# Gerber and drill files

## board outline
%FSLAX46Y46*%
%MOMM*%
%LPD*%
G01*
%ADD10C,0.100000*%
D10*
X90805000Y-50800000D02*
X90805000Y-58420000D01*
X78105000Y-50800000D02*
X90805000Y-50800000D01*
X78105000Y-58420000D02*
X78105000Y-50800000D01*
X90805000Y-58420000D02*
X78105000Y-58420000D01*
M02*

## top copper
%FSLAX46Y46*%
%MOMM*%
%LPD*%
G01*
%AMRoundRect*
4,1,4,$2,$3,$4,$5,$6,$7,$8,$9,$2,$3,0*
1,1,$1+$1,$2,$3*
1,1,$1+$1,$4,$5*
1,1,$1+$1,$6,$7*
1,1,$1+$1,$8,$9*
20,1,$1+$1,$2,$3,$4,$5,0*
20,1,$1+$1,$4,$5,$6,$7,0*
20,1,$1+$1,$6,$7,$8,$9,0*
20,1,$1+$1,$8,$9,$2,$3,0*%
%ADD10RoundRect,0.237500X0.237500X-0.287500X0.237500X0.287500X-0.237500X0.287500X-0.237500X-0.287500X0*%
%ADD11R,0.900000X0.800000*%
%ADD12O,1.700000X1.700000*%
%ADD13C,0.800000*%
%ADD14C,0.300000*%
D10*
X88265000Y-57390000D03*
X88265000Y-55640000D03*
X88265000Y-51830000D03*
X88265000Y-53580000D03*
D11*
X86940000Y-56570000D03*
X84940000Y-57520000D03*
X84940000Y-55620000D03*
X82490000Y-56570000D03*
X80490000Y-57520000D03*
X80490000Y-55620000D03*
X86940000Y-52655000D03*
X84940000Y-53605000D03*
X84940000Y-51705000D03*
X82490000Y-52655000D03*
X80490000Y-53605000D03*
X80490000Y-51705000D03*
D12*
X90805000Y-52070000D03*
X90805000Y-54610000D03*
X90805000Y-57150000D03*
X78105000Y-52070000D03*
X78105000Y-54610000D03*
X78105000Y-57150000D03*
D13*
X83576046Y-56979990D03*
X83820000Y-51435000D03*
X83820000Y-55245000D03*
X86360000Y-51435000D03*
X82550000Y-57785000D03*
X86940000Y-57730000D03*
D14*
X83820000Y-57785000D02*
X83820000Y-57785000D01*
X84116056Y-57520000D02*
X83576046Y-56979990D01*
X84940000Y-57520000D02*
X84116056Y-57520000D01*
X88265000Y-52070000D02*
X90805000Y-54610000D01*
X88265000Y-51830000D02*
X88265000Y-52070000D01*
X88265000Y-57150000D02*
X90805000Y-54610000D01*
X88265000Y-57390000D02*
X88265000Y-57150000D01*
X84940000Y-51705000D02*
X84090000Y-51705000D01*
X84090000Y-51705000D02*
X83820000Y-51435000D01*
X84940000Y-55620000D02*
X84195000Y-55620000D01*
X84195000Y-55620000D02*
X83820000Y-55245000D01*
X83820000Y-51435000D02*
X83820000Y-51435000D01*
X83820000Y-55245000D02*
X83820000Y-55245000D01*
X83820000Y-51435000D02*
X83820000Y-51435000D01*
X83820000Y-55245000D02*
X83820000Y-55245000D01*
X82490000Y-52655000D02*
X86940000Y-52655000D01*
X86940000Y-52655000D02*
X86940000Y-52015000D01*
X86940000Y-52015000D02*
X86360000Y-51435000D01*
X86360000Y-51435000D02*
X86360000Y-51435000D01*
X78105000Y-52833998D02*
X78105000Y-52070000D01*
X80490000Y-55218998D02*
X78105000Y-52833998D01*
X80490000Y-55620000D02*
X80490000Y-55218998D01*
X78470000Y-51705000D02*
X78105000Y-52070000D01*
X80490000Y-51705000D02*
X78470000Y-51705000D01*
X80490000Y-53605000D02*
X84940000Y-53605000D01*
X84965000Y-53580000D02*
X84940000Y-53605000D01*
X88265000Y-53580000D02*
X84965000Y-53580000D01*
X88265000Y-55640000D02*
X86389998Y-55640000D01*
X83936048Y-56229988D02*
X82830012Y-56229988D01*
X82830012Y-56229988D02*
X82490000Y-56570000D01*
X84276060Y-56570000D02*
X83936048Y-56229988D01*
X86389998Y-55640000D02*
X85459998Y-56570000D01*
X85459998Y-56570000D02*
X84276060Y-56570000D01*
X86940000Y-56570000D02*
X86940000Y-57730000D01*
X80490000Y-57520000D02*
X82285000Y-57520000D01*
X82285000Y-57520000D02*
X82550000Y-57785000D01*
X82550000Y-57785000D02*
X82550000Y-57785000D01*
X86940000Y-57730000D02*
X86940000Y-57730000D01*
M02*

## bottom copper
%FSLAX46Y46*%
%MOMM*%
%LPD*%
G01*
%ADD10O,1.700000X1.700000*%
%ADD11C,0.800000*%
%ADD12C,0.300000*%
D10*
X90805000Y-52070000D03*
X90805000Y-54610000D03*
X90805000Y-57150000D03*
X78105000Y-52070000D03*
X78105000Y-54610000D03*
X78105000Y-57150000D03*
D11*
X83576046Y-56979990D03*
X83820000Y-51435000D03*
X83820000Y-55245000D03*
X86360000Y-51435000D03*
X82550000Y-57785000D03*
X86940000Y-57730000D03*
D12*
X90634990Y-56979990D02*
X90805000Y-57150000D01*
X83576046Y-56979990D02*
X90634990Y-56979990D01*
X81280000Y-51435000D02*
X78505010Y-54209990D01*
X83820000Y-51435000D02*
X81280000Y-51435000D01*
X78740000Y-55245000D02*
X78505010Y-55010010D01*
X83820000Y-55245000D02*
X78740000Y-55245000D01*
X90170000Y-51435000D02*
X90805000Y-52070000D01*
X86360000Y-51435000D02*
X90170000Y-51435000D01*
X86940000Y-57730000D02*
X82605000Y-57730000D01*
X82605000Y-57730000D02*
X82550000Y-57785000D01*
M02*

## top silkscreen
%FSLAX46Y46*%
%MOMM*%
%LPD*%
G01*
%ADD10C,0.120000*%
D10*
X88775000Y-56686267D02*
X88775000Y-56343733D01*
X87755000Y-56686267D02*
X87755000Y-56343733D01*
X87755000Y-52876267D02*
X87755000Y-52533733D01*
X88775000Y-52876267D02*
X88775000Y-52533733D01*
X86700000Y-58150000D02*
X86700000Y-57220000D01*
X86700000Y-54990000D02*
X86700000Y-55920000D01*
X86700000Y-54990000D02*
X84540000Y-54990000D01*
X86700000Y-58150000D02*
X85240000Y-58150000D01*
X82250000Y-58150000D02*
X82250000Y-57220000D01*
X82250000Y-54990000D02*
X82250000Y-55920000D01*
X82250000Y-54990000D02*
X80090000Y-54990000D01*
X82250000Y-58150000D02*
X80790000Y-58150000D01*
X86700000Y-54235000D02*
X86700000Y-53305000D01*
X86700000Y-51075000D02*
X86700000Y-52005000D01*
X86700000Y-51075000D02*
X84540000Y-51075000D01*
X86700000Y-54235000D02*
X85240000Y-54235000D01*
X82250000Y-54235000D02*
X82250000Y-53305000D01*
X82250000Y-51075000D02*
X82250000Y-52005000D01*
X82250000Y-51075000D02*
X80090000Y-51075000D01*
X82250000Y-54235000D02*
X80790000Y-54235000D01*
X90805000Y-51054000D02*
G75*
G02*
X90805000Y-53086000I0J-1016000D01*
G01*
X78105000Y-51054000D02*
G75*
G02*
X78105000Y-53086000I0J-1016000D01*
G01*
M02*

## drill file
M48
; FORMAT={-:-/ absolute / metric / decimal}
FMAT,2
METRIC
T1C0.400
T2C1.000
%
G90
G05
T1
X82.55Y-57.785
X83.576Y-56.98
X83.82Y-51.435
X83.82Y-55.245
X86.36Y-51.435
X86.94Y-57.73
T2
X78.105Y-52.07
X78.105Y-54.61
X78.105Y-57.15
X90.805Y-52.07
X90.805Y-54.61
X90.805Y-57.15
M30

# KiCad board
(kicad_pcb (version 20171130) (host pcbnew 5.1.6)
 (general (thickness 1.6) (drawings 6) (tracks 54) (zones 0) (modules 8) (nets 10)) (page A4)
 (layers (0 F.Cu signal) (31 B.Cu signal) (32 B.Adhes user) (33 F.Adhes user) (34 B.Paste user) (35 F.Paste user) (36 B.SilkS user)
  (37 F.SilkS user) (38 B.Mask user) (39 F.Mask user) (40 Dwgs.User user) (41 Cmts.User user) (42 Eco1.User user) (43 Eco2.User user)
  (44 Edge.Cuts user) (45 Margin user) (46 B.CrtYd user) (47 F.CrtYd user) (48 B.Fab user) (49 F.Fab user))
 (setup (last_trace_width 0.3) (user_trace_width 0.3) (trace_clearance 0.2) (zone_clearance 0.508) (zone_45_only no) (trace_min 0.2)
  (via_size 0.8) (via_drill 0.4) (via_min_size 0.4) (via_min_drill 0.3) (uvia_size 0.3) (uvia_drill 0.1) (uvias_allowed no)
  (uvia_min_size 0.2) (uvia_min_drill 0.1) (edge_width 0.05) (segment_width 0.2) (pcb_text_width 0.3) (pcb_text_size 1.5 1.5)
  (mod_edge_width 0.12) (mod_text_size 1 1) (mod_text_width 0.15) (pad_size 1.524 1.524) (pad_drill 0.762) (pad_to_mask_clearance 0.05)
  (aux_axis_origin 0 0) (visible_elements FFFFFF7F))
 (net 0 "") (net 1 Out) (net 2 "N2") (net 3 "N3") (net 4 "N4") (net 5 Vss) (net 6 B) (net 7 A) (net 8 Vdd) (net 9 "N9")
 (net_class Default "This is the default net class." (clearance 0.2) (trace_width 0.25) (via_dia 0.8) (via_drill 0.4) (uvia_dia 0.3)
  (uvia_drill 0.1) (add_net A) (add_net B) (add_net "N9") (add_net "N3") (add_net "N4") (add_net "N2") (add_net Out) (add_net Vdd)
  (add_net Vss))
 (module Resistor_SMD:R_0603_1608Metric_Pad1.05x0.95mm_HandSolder (layer F.Cu) (at 88.265 56.515 90)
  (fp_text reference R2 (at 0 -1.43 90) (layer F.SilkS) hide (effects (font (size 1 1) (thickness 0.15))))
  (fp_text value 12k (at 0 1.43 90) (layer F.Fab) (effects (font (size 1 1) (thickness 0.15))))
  (fp_line (start -0.171267 0.51) (end 0.171267 0.51) (layer F.SilkS) (width 0.12))
  (fp_line (start -0.171267 -0.51) (end 0.171267 -0.51) (layer F.SilkS) (width 0.12))
  (pad 1 smd roundrect (at -0.875 0 90) (size 1.05 0.95) (layers F.Cu F.Paste F.Mask) (roundrect_rratio 0.25) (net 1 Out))
  (pad 2 smd roundrect (at 0.875 0 90) (size 1.05 0.95) (layers F.Cu F.Paste F.Mask) (roundrect_rratio 0.25) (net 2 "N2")))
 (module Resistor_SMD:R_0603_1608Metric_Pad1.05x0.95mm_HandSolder (layer F.Cu) (at 88.265 52.705 90)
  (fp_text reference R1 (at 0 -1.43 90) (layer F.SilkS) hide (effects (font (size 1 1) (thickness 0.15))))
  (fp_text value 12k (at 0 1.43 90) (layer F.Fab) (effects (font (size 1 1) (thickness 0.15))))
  (fp_line (start -0.171267 -0.51) (end 0.171267 -0.51) (layer F.SilkS) (width 0.12))
  (fp_line (start -0.171267 0.51) (end 0.171267 0.51) (layer F.SilkS) (width 0.12))
  (pad 2 smd roundrect (at 0.875 0 90) (size 1.05 0.95) (layers F.Cu F.Paste F.Mask) (roundrect_rratio 0.25) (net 1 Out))
  (pad 1 smd roundrect (at -0.875 0 90) (size 1.05 0.95) (layers F.Cu F.Paste F.Mask) (roundrect_rratio 0.25) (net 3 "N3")))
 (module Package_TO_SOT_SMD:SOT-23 (layer F.Cu) (at 85.94 56.57)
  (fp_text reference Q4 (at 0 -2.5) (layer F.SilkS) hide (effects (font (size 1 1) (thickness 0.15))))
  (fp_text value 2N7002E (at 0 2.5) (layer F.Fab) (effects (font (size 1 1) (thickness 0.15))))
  (fp_line (start 0.76 1.58) (end 0.76 0.65) (layer F.SilkS) (width 0.12))
  (fp_line (start 0.76 -1.58) (end 0.76 -0.65) (layer F.SilkS) (width 0.12))
  (fp_line (start 0.76 -1.58) (end -1.4 -1.58) (layer F.SilkS) (width 0.12))
  (fp_line (start 0.76 1.58) (end -0.7 1.58) (layer F.SilkS) (width 0.12))
  (pad 3 smd rect (at 1 0) (size 0.9 0.8) (layers F.Cu F.Paste F.Mask) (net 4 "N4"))
  (pad 2 smd rect (at -1 0.95) (size 0.9 0.8) (layers F.Cu F.Paste F.Mask) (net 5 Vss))
  (pad 1 smd rect (at -1 -0.95) (size 0.9 0.8) (layers F.Cu F.Paste F.Mask) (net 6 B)))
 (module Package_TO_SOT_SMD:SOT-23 (layer F.Cu) (at 81.49 56.57)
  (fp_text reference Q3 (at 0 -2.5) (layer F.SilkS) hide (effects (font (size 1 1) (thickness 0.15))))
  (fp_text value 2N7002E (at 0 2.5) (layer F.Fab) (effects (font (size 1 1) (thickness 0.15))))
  (fp_line (start 0.76 1.58) (end 0.76 0.65) (layer F.SilkS) (width 0.12))
  (fp_line (start 0.76 -1.58) (end 0.76 -0.65) (layer F.SilkS) (width 0.12))
  (fp_line (start 0.76 -1.58) (end -1.4 -1.58) (layer F.SilkS) (width 0.12))
  (fp_line (start 0.76 1.58) (end -0.7 1.58) (layer F.SilkS) (width 0.12))
  (pad 3 smd rect (at 1 0) (size 0.9 0.8) (layers F.Cu F.Paste F.Mask) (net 2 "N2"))
  (pad 2 smd rect (at -1 0.95) (size 0.9 0.8) (layers F.Cu F.Paste F.Mask) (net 4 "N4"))
  (pad 1 smd rect (at -1 -0.95) (size 0.9 0.8) (layers F.Cu F.Paste F.Mask) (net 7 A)))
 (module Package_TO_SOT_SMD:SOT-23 (layer F.Cu) (at 85.94 52.655)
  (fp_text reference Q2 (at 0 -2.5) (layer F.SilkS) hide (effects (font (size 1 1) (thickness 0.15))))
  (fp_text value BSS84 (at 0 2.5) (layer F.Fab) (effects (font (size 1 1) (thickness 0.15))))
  (fp_line (start 0.76 1.58) (end 0.76 0.65) (layer F.SilkS) (width 0.12))
  (fp_line (start 0.76 -1.58) (end 0.76 -0.65) (layer F.SilkS) (width 0.12))
  (fp_line (start 0.76 -1.58) (end -1.4 -1.58) (layer F.SilkS) (width 0.12))
  (fp_line (start 0.76 1.58) (end -0.7 1.58) (layer F.SilkS) (width 0.12))
  (pad 3 smd rect (at 1 0) (size 0.9 0.8) (layers F.Cu F.Paste F.Mask) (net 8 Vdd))
  (pad 2 smd rect (at -1 0.95) (size 0.9 0.8) (layers F.Cu F.Paste F.Mask) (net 3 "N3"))
  (pad 1 smd rect (at -1 -0.95) (size 0.9 0.8) (layers F.Cu F.Paste F.Mask) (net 6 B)))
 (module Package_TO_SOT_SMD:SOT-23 (layer F.Cu) (at 81.49 52.655)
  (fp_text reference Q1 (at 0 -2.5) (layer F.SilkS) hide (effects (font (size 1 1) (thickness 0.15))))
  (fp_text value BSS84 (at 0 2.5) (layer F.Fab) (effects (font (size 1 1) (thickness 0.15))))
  (fp_line (start 0.76 1.58) (end 0.76 0.65) (layer F.SilkS) (width 0.12))
  (fp_line (start 0.76 -1.58) (end 0.76 -0.65) (layer F.SilkS) (width 0.12))
  (fp_line (start 0.76 -1.58) (end -1.4 -1.58) (layer F.SilkS) (width 0.12))
  (fp_line (start 0.76 1.58) (end -0.7 1.58) (layer F.SilkS) (width 0.12))
  (pad 3 smd rect (at 1 0) (size 0.9 0.8) (layers F.Cu F.Paste F.Mask) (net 8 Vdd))
  (pad 2 smd rect (at -1 0.95) (size 0.9 0.8) (layers F.Cu F.Paste F.Mask) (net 3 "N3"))
  (pad 1 smd rect (at -1 -0.95) (size 0.9 0.8) (layers F.Cu F.Paste F.Mask) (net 7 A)))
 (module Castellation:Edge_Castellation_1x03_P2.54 (layer F.Cu) (at 90.805 52.07)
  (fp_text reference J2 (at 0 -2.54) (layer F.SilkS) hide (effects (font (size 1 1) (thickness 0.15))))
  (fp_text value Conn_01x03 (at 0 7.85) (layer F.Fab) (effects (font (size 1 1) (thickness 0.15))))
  (fp_arc (start 0 0) (end 0 1.016) (angle -180) (layer F.SilkS) (width 0.12))
  (pad 1 thru_hole oval (at 0 0) (size 1.7 1.7) (drill 1) (layers *.Cu *.Mask) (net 8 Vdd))
  (pad 2 thru_hole oval (at 0 2.54) (size 1.7 1.7) (drill 1) (layers *.Cu *.Mask) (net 1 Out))
  (pad 3 thru_hole oval (at 0 5.08) (size 1.7 1.7) (drill 1) (layers *.Cu *.Mask) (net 5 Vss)))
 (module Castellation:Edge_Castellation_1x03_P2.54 (layer F.Cu) (at 78.105 52.07)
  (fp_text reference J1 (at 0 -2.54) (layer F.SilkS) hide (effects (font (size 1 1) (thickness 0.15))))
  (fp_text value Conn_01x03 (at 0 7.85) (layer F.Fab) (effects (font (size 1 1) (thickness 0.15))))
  (fp_arc (start 0 0) (end 0 1.016) (angle -180) (layer F.SilkS) (width 0.12))
  (pad 1 thru_hole oval (at 0 0) (size 1.7 1.7) (drill 1) (layers *.Cu *.Mask) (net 7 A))
  (pad 2 thru_hole oval (at 0 2.54) (size 1.7 1.7) (drill 1) (layers *.Cu *.Mask) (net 6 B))
  (pad 3 thru_hole oval (at 0 5.08) (size 1.7 1.7) (drill 1) (layers *.Cu *.Mask) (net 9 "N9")))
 (gr_line (start 90.805 50.8) (end 90.805 58.42) (layer Edge.Cuts) (width 0.1))
 (gr_line (start 78.105 50.8) (end 90.805 50.8) (layer Edge.Cuts) (width 0.1))
 (gr_line (start 78.105 58.42) (end 78.105 50.8) (layer Edge.Cuts) (width 0.1))
 (gr_line (start 90.805 58.42) (end 78.105 58.42) (layer Edge.Cuts) (width 0.1))
 (segment (start 83.82 57.785) (end 83.82 57.785) (width 0.3) (layer F.Cu) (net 5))
 (segment (start 84.116056 57.52) (end 83.576046 56.97999) (width 0.3) (layer F.Cu) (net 5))
 (segment (start 84.94 57.52) (end 84.116056 57.52) (width 0.3) (layer F.Cu) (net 5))
 (via (at 83.576046 56.97999) (size 0.8) (drill 0.4) (layers F.Cu B.Cu) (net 5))
 (segment (start 90.63499 56.97999) (end 90.805 57.15) (width 0.3) (layer B.Cu) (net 5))
 (segment (start 83.576046 56.97999) (end 90.63499 56.97999) (width 0.3) (layer B.Cu) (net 5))
 (segment (start 88.265 52.07) (end 90.805 54.61) (width 0.3) (layer F.Cu) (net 1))
 (segment (start 88.265 51.83) (end 88.265 52.07) (width 0.3) (layer F.Cu) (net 1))
 (segment (start 88.265 57.15) (end 90.805 54.61) (width 0.3) (layer F.Cu) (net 1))
 (segment (start 88.265 57.39) (end 88.265 57.15) (width 0.3) (layer F.Cu) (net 1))
 (segment (start 84.94 51.705) (end 84.09 51.705) (width 0.3) (layer F.Cu) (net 6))
 (segment (start 84.09 51.705) (end 83.82 51.435) (width 0.3) (layer F.Cu) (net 6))
 (segment (start 84.94 55.62) (end 84.195 55.62) (width 0.3) (layer F.Cu) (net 6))
 (segment (start 84.195 55.62) (end 83.82 55.245) (width 0.3) (layer F.Cu) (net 6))
 (segment (start 83.82 51.435) (end 83.82 51.435) (width 0.3) (layer F.Cu) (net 6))
 (segment (start 83.82 55.245) (end 83.82 55.245) (width 0.3) (layer F.Cu) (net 6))
 (segment (start 83.82 51.435) (end 83.82 51.435) (width 0.3) (layer F.Cu) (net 6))
 (via (at 83.82 51.435) (size 0.8) (drill 0.4) (layers F.Cu B.Cu) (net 6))
 (segment (start 83.82 55.245) (end 83.82 55.245) (width 0.3) (layer F.Cu) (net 6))
 (via (at 83.82 55.245) (size 0.8) (drill 0.4) (layers F.Cu B.Cu) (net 6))
 (segment (start 81.28 51.435) (end 78.50501 54.20999) (width 0.3) (layer B.Cu) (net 6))
 (segment (start 83.82 51.435) (end 81.28 51.435) (width 0.3) (layer B.Cu) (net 6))
 (segment (start 78.74 55.245) (end 78.50501 55.01001) (width 0.3) (layer B.Cu) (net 6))
 (segment (start 83.82 55.245) (end 78.74 55.245) (width 0.3) (layer B.Cu) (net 6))
 (segment (start 82.49 52.655) (end 86.94 52.655) (width 0.3) (layer F.Cu) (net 8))
 (segment (start 86.94 52.655) (end 86.94 52.015) (width 0.3) (layer F.Cu) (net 8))
 (segment (start 86.94 52.015) (end 86.36 51.435) (width 0.3) (layer F.Cu) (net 8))
 (segment (start 86.36 51.435) (end 86.36 51.435) (width 0.3) (layer F.Cu) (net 8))
 (via (at 86.36 51.435) (size 0.8) (drill 0.4) (layers F.Cu B.Cu) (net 8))
 (segment (start 90.17 51.435) (end 90.805 52.07) (width 0.3) (layer B.Cu) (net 8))
 (segment (start 86.36 51.435) (end 90.17 51.435) (width 0.3) (layer B.Cu) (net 8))
 (segment (start 78.105 52.833998) (end 78.105 52.07) (width 0.3) (layer F.Cu) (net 7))
 (segment (start 80.49 55.218998) (end 78.105 52.833998) (width 0.3) (layer F.Cu) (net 7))
 (segment (start 80.49 55.62) (end 80.49 55.218998) (width 0.3) (layer F.Cu) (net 7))
 (segment (start 78.47 51.705) (end 78.105 52.07) (width 0.3) (layer F.Cu) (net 7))
 (segment (start 80.49 51.705) (end 78.47 51.705) (width 0.3) (layer F.Cu) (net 7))
 (segment (start 80.49 53.605) (end 84.94 53.605) (width 0.3) (layer F.Cu) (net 3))
 (segment (start 84.965 53.58) (end 84.94 53.605) (width 0.3) (layer F.Cu) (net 3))
 (segment (start 88.265 53.58) (end 84.965 53.58) (width 0.3) (layer F.Cu) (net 3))
 (segment (start 88.265 55.64) (end 86.389998 55.64) (width 0.3) (layer F.Cu) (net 2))
 (segment (start 83.936048 56.229988) (end 82.830012 56.229988) (width 0.3) (layer F.Cu) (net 2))
 (segment (start 82.830012 56.229988) (end 82.49 56.57) (width 0.3) (layer F.Cu) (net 2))
 (segment (start 84.27606 56.57) (end 83.936048 56.229988) (width 0.3) (layer F.Cu) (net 2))
 (segment (start 86.389998 55.64) (end 85.459998 56.57) (width 0.3) (layer F.Cu) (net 2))
 (segment (start 85.459998 56.57) (end 84.27606 56.57) (width 0.3) (layer F.Cu) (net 2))
 (segment (start 86.94 56.57) (end 86.94 57.73) (width 0.3) (layer F.Cu) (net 4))
 (segment (start 80.49 57.52) (end 82.285 57.52) (width 0.3) (layer F.Cu) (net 4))
 (segment (start 82.285 57.52) (end 82.55 57.785) (width 0.3) (layer F.Cu) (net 4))
 (segment (start 82.55 57.785) (end 82.55 57.785) (width 0.3) (layer F.Cu) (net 4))
 (via (at 82.55 57.785) (size 0.8) (drill 0.4) (layers F.Cu B.Cu) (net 4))
 (segment (start 86.94 57.73) (end 86.94 57.73) (width 0.3) (layer F.Cu) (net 4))
 (via (at 86.94 57.73) (size 0.8) (drill 0.4) (layers F.Cu B.Cu) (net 4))
 (segment (start 86.94 57.73) (end 82.605 57.73) (width 0.3) (layer B.Cu) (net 4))
 (segment (start 82.605 57.73) (end 82.55 57.785) (width 0.3) (layer B.Cu) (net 4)))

